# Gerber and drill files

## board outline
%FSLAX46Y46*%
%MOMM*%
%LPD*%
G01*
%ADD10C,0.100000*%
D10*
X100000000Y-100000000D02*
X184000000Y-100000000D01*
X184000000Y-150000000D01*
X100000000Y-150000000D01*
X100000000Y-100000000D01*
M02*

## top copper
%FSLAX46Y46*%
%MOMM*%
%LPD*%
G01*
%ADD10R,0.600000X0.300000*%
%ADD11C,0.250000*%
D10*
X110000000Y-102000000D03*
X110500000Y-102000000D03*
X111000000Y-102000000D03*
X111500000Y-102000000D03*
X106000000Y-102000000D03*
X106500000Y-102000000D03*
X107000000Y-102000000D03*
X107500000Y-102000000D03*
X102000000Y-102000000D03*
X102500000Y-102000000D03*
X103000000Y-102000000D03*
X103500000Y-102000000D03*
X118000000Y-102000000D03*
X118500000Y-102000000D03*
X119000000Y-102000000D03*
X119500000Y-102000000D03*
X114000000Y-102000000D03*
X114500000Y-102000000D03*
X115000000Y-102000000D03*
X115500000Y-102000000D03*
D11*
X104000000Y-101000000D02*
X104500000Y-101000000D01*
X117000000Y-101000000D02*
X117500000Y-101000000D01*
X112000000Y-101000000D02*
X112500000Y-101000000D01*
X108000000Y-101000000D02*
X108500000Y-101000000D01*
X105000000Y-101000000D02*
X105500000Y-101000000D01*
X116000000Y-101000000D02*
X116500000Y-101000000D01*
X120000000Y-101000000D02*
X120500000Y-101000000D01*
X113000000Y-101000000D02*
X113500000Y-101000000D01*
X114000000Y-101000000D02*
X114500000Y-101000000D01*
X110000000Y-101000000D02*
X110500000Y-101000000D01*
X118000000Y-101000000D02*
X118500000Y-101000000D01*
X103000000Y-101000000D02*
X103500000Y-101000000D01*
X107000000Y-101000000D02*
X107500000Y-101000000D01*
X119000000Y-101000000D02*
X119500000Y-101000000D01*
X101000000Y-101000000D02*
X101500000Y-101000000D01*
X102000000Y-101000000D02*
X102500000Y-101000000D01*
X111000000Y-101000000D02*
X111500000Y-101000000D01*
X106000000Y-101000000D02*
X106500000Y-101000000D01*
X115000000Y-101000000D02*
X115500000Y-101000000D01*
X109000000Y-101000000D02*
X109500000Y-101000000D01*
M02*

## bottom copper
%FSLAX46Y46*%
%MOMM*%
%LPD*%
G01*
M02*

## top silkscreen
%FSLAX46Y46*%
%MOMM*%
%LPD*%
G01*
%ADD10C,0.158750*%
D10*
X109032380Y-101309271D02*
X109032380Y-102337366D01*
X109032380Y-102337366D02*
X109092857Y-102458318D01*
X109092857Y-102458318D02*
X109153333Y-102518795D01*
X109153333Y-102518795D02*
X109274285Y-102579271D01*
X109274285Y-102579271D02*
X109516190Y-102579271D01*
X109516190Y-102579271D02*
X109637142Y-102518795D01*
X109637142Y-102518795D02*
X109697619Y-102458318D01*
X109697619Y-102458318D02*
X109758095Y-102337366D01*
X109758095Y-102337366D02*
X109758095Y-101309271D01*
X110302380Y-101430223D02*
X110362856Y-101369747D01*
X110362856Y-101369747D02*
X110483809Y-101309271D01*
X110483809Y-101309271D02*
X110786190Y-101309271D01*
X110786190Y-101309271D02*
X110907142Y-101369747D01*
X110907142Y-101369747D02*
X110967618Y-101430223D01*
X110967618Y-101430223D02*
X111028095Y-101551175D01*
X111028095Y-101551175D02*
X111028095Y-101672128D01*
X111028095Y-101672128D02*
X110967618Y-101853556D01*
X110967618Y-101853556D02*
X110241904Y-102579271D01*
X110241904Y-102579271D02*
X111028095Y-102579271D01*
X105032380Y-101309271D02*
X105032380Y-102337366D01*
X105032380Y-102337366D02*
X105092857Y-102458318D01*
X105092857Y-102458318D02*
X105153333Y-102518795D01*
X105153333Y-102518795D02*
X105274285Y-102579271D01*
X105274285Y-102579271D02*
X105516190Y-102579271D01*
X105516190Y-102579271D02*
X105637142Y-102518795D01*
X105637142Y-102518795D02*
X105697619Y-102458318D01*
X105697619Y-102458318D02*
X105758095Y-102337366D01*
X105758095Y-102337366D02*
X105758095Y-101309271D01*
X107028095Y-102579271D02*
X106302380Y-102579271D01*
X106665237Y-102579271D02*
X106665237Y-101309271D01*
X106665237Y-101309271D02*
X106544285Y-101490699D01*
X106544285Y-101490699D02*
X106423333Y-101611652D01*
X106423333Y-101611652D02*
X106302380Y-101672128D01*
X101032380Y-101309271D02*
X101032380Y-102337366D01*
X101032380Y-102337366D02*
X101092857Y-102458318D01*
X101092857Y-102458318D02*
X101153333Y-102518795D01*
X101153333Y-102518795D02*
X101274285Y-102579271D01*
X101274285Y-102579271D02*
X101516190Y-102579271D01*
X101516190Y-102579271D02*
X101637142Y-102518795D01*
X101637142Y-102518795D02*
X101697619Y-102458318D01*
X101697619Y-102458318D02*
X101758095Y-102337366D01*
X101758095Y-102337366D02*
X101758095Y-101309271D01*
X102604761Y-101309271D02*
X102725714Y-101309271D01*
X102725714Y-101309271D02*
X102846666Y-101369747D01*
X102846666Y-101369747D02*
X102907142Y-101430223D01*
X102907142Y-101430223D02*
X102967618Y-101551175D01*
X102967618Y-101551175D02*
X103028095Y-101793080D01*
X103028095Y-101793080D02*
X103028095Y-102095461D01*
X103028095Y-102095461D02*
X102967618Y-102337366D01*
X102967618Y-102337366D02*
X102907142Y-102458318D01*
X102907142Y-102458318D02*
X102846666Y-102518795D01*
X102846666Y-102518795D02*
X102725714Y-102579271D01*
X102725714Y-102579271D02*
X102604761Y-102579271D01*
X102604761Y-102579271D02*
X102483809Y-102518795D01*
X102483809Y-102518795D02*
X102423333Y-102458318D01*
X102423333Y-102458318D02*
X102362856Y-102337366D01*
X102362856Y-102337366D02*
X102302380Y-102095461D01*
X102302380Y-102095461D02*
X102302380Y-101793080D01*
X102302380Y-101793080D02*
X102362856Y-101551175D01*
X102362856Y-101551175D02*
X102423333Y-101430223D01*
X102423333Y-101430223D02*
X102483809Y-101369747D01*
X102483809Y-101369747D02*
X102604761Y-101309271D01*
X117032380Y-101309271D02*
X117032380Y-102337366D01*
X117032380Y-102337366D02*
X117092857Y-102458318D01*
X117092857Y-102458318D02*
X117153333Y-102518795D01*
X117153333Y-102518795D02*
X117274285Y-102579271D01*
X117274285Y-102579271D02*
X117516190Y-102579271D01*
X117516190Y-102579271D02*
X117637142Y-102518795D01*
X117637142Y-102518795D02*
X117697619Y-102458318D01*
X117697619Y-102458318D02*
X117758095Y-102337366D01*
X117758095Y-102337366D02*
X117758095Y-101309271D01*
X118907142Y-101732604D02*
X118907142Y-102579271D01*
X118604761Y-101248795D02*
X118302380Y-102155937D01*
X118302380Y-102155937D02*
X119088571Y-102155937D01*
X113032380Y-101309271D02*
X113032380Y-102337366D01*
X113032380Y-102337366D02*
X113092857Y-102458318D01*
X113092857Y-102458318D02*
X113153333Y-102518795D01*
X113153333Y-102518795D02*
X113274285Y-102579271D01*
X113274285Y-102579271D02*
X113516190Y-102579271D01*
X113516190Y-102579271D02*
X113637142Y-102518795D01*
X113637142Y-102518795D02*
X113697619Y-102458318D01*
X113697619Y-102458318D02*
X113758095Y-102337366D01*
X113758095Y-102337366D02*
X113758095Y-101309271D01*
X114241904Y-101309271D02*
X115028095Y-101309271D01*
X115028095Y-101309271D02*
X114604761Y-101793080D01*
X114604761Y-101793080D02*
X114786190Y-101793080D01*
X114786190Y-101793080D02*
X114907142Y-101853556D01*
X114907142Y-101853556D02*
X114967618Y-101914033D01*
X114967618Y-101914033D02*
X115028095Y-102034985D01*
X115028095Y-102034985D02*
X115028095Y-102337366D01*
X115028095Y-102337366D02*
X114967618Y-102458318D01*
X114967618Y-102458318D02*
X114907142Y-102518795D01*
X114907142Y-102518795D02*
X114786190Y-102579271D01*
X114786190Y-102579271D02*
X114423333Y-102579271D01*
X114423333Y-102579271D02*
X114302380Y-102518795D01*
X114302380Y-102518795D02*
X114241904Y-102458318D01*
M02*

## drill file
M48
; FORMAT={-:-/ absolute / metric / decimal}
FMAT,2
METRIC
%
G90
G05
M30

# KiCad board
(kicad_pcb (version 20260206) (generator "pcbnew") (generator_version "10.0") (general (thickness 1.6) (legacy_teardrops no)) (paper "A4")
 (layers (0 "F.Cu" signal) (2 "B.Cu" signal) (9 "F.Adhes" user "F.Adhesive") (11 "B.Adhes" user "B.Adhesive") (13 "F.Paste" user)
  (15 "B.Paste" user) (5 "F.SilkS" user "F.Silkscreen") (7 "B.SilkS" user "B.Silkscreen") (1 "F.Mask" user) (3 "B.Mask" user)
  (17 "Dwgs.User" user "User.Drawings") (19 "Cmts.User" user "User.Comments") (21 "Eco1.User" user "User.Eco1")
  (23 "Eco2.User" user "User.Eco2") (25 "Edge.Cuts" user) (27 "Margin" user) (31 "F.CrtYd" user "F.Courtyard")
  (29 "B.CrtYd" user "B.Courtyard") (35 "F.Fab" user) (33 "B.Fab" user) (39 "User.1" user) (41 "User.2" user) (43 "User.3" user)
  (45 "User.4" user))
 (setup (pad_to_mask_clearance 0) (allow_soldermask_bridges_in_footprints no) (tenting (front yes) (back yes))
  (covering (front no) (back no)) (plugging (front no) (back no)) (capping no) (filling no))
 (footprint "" (layer "F.Cu") (at 110 102)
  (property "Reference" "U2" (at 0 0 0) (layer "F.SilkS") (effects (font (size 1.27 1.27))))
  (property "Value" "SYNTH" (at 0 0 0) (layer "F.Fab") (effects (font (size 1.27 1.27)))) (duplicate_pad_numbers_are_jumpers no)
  (pad "1" smd rect (at 0 0) (size 0.6 0.3) (layers "F.Cu" "F.Mask" "F.Paste") (thermal_bridge_angle 45))
  (pad "2" smd rect (at 0.5 0) (size 0.6 0.3) (layers "F.Cu" "F.Mask" "F.Paste") (thermal_bridge_angle 45))
  (pad "3" smd rect (at 1 0) (size 0.6 0.3) (layers "F.Cu" "F.Mask" "F.Paste") (thermal_bridge_angle 45))
  (pad "4" smd rect (at 1.5 0) (size 0.6 0.3) (layers "F.Cu" "F.Mask" "F.Paste") (thermal_bridge_angle 45)))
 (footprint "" (layer "F.Cu") (at 106 102)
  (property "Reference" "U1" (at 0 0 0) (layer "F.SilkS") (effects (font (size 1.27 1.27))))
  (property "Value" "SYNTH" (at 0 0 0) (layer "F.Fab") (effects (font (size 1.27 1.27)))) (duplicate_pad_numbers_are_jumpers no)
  (pad "1" smd rect (at 0 0) (size 0.6 0.3) (layers "F.Cu" "F.Mask" "F.Paste") (thermal_bridge_angle 45))
  (pad "2" smd rect (at 0.5 0) (size 0.6 0.3) (layers "F.Cu" "F.Mask" "F.Paste") (thermal_bridge_angle 45))
  (pad "3" smd rect (at 1 0) (size 0.6 0.3) (layers "F.Cu" "F.Mask" "F.Paste") (thermal_bridge_angle 45))
  (pad "4" smd rect (at 1.5 0) (size 0.6 0.3) (layers "F.Cu" "F.Mask" "F.Paste") (thermal_bridge_angle 45)))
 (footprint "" (layer "F.Cu") (at 102 102)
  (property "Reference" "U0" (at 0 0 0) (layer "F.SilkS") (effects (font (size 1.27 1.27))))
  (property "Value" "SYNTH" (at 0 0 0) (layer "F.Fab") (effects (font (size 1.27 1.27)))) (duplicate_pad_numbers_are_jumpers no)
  (pad "1" smd rect (at 0 0) (size 0.6 0.3) (layers "F.Cu" "F.Mask" "F.Paste") (thermal_bridge_angle 45))
  (pad "2" smd rect (at 0.5 0) (size 0.6 0.3) (layers "F.Cu" "F.Mask" "F.Paste") (thermal_bridge_angle 45))
  (pad "3" smd rect (at 1 0) (size 0.6 0.3) (layers "F.Cu" "F.Mask" "F.Paste") (thermal_bridge_angle 45))
  (pad "4" smd rect (at 1.5 0) (size 0.6 0.3) (layers "F.Cu" "F.Mask" "F.Paste") (thermal_bridge_angle 45)))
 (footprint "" (layer "F.Cu") (at 118 102)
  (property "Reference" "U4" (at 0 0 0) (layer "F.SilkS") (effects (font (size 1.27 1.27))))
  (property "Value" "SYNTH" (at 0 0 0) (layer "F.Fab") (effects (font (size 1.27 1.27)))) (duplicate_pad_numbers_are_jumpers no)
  (pad "1" smd rect (at 0 0) (size 0.6 0.3) (layers "F.Cu" "F.Mask" "F.Paste") (thermal_bridge_angle 45))
  (pad "2" smd rect (at 0.5 0) (size 0.6 0.3) (layers "F.Cu" "F.Mask" "F.Paste") (thermal_bridge_angle 45))
  (pad "3" smd rect (at 1 0) (size 0.6 0.3) (layers "F.Cu" "F.Mask" "F.Paste") (thermal_bridge_angle 45))
  (pad "4" smd rect (at 1.5 0) (size 0.6 0.3) (layers "F.Cu" "F.Mask" "F.Paste") (thermal_bridge_angle 45)))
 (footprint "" (layer "F.Cu") (at 114 102)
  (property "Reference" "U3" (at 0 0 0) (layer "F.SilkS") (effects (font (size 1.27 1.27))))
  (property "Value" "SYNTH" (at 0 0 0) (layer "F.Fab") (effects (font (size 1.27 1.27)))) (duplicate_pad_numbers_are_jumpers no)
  (pad "1" smd rect (at 0 0) (size 0.6 0.3) (layers "F.Cu" "F.Mask" "F.Paste") (thermal_bridge_angle 45))
  (pad "2" smd rect (at 0.5 0) (size 0.6 0.3) (layers "F.Cu" "F.Mask" "F.Paste") (thermal_bridge_angle 45))
  (pad "3" smd rect (at 1 0) (size 0.6 0.3) (layers "F.Cu" "F.Mask" "F.Paste") (thermal_bridge_angle 45))
  (pad "4" smd rect (at 1.5 0) (size 0.6 0.3) (layers "F.Cu" "F.Mask" "F.Paste") (thermal_bridge_angle 45)))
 (gr_rect (start 100 100) (end 184 150) (stroke (width 0.1) (type default)) (fill no) (layer "Edge.Cuts"))
 (segment (start 104 101) (end 104.5 101) (width 0.25) (layer "F.Cu") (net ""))
 (segment (start 117 101) (end 117.5 101) (width 0.25) (layer "F.Cu") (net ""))
 (segment (start 112 101) (end 112.5 101) (width 0.25) (layer "F.Cu") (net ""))
 (segment (start 108 101) (end 108.5 101) (width 0.25) (layer "F.Cu") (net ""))
 (segment (start 105 101) (end 105.5 101) (width 0.25) (layer "F.Cu") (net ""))
 (segment (start 116 101) (end 116.5 101) (width 0.25) (layer "F.Cu") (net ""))
 (segment (start 120 101) (end 120.5 101) (width 0.25) (layer "F.Cu") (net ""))
 (segment (start 113 101) (end 113.5 101) (width 0.25) (layer "F.Cu") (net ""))
 (segment (start 114 101) (end 114.5 101) (width 0.25) (layer "F.Cu") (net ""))
 (segment (start 110 101) (end 110.5 101) (width 0.25) (layer "F.Cu") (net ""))
 (segment (start 118 101) (end 118.5 101) (width 0.25) (layer "F.Cu") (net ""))
 (segment (start 103 101) (end 103.5 101) (width 0.25) (layer "F.Cu") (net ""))
 (segment (start 107 101) (end 107.5 101) (width 0.25) (layer "F.Cu") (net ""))
 (segment (start 119 101) (end 119.5 101) (width 0.25) (layer "F.Cu") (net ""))
 (segment (start 101 101) (end 101.5 101) (width 0.25) (layer "F.Cu") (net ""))
 (segment (start 102 101) (end 102.5 101) (width 0.25) (layer "F.Cu") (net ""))
 (segment (start 111 101) (end 111.5 101) (width 0.25) (layer "F.Cu") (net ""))
 (segment (start 106 101) (end 106.5 101) (width 0.25) (layer "F.Cu") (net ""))
 (segment (start 115 101) (end 115.5 101) (width 0.25) (layer "F.Cu") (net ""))
 (segment (start 109 101) (end 109.5 101) (width 0.25) (layer "F.Cu") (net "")))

